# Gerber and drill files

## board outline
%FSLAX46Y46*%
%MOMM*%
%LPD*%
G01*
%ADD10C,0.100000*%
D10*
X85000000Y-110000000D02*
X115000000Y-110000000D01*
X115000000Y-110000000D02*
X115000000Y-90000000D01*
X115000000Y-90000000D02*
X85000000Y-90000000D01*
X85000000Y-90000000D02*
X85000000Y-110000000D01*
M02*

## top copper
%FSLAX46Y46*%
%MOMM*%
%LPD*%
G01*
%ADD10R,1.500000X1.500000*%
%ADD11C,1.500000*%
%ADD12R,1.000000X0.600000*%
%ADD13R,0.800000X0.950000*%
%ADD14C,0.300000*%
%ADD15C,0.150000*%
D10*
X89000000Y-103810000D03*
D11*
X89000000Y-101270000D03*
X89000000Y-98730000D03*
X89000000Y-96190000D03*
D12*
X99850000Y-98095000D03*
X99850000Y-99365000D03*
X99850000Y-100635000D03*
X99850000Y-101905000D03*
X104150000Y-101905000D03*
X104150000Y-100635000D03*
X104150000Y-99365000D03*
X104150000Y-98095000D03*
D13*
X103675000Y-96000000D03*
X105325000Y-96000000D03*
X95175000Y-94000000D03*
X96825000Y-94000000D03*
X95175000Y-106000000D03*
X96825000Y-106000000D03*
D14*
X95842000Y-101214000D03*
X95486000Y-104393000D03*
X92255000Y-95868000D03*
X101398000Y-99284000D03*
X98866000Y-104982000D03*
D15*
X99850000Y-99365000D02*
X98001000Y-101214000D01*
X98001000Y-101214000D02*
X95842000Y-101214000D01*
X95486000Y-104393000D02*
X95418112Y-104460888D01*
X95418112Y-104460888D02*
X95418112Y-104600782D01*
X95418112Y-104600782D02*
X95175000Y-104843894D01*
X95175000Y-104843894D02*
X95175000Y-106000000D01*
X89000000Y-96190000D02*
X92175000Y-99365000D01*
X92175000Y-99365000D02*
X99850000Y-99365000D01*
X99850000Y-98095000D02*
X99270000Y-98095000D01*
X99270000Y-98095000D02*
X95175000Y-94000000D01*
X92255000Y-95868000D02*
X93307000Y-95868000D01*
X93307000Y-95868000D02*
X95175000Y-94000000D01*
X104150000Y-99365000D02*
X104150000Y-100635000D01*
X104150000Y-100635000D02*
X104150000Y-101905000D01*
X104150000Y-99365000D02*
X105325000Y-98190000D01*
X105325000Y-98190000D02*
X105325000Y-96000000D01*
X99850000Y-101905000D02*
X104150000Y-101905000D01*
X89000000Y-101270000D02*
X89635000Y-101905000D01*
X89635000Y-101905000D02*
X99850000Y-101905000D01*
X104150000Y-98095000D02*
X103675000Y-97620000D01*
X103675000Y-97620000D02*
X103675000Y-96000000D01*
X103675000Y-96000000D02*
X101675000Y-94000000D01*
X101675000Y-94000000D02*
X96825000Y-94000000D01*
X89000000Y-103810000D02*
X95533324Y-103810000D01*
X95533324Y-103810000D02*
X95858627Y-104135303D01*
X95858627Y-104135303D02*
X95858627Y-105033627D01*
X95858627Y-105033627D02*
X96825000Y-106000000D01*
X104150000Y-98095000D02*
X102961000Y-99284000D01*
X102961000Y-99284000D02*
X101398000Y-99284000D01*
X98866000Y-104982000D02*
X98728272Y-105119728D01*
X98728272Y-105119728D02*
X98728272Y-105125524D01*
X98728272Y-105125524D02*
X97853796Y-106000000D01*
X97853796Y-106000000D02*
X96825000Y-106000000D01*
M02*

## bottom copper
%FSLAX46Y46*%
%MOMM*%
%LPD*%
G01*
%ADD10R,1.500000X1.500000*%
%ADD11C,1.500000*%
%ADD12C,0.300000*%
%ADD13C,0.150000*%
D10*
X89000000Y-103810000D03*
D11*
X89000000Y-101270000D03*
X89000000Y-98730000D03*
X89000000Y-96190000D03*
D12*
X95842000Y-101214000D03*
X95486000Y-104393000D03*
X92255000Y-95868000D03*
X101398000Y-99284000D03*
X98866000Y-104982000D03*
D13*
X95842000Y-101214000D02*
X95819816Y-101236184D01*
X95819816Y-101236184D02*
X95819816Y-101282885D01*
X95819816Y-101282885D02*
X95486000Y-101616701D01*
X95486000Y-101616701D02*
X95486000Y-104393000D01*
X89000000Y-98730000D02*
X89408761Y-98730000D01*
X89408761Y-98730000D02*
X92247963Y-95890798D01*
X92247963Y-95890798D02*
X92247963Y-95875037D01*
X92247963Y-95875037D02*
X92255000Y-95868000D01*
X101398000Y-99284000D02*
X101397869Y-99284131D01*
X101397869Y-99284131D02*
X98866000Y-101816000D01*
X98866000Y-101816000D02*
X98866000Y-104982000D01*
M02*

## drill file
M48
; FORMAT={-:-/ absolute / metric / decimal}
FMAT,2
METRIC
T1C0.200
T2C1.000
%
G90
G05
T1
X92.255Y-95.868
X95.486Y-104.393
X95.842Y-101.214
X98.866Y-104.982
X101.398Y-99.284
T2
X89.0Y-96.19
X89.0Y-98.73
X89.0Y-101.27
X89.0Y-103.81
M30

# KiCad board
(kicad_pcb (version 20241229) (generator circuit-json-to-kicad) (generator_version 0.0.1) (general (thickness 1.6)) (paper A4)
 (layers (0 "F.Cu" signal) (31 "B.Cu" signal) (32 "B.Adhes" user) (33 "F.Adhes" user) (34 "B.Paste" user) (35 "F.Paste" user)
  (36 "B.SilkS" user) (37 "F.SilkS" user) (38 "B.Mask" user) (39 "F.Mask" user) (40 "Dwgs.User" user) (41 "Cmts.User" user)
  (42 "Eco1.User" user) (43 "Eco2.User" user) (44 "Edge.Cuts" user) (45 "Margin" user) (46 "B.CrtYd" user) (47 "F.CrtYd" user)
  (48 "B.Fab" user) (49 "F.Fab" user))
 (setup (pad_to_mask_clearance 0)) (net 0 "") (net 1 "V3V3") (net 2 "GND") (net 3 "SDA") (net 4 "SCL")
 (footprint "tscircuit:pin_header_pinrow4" (layer F.Cu) (at 89 100 90)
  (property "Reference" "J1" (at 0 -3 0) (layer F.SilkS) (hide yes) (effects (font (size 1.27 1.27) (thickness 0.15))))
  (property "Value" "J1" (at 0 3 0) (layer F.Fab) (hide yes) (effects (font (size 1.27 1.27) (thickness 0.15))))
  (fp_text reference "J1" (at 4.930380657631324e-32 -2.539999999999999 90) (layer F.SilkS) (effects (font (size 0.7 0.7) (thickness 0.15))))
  (pad "1" thru_hole rect (at -3.81 2.3329521523757077e-16 90) (size 1.5 1.5) (drill 1) (layers *.Cu *.Mask) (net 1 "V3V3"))
  (pad "2" thru_hole circle (at -1.27 7.776507174585693e-17 0) (size 1.5 1.5) (drill 1) (layers *.Cu *.Mask) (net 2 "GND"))
  (pad "3" thru_hole circle (at 1.27 -7.776507174585693e-17 0) (size 1.5 1.5) (drill 1) (layers *.Cu *.Mask) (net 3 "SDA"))
  (pad "4" thru_hole circle (at 3.81 -2.3329521523757077e-16 0) (size 1.5 1.5) (drill 1) (layers *.Cu *.Mask) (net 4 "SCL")))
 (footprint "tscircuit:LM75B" (layer F.Cu) (at 102 100 0)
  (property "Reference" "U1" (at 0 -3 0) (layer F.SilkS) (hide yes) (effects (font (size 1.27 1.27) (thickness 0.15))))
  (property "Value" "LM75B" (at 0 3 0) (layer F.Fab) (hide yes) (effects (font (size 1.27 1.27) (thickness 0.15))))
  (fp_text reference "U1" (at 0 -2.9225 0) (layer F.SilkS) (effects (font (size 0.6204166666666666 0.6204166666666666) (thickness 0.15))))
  (pad "1" smd rect (at -2.15 -1.905 0) (size 1 0.6) (layers F.Cu F.Paste F.Mask) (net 3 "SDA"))
  (pad "2" smd rect (at -2.15 -0.635 0) (size 1 0.6) (layers F.Cu F.Paste F.Mask) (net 4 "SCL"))
  (pad "3" smd rect (at -2.15 0.635 0) (size 1 0.6) (layers F.Cu F.Paste F.Mask))
  (pad "4" smd rect (at -2.15 1.905 0) (size 1 0.6) (layers F.Cu F.Paste F.Mask) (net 2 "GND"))
  (pad "5" smd rect (at 2.1500000000000004 1.905 0) (size 1 0.6) (layers F.Cu F.Paste F.Mask) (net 2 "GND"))
  (pad "6" smd rect (at 2.1500000000000004 0.635 0) (size 1 0.6) (layers F.Cu F.Paste F.Mask) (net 2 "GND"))
  (pad "7" smd rect (at 2.1500000000000004 -0.635 0) (size 1 0.6) (layers F.Cu F.Paste F.Mask) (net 2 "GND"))
  (pad "8" smd rect (at 2.1500000000000004 -1.905 0) (size 1 0.6) (layers F.Cu F.Paste F.Mask) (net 1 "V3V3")))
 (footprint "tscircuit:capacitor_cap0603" (layer F.Cu) (at 104.5 96 0)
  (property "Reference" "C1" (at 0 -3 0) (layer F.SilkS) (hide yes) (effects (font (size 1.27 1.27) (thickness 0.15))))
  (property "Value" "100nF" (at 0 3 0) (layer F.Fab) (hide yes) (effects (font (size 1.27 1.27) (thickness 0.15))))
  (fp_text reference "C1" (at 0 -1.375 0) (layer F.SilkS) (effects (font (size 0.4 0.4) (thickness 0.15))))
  (pad "1" smd rect (at -0.8250000000000002 0 0) (size 0.8 0.95) (layers F.Cu F.Paste F.Mask) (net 1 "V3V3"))
  (pad "2" smd rect (at 0.8250000000000002 0 0) (size 0.8 0.95) (layers F.Cu F.Paste F.Mask) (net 2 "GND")))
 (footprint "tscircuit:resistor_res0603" (layer F.Cu) (at 96 94 0)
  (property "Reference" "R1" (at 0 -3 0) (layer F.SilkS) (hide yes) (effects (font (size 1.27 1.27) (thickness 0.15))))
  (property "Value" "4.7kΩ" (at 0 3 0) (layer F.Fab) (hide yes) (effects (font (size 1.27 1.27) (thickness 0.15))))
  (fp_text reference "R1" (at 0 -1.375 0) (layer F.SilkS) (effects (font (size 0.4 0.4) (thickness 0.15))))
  (pad "1" smd rect (at -0.8250000000000002 0 0) (size 0.8 0.95) (layers F.Cu F.Paste F.Mask) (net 3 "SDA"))
  (pad "2" smd rect (at 0.8250000000000002 0 0) (size 0.8 0.95) (layers F.Cu F.Paste F.Mask) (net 1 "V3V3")))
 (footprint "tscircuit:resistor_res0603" (layer F.Cu) (at 96 106 0)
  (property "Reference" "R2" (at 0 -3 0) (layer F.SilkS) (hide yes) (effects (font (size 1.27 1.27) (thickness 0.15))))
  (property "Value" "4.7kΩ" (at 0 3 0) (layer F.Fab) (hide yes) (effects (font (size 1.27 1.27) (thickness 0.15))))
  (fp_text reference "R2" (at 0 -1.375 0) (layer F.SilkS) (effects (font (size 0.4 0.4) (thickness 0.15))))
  (pad "1" smd rect (at -0.8250000000000002 0 0) (size 0.8 0.95) (layers F.Cu F.Paste F.Mask) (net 4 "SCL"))
  (pad "2" smd rect (at 0.8250000000000002 0 0) (size 0.8 0.95) (layers F.Cu F.Paste F.Mask) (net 1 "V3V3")))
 (segment (start 99.85 99.365) (end 98.001 101.214) (width 0.15) (layer F.Cu) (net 4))
 (segment (start 98.001 101.214) (end 95.842 101.214) (width 0.15) (layer F.Cu) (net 4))
 (segment (start 95.842 101.214) (end 95.81981559401727 101.23618440598273) (width 0.15) (layer B.Cu) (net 4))
 (segment (start 95.81981559401727 101.23618440598273) (end 95.81981559401727 101.28288511764556) (width 0.15) (layer B.Cu) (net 4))
 (segment (start 95.81981559401727 101.28288511764556) (end 95.486 101.61670071166283) (width 0.15) (layer B.Cu) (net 4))
 (segment (start 95.486 101.61670071166283) (end 95.486 104.393) (width 0.15) (layer B.Cu) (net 4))
 (segment (start 95.486 104.393) (end 95.41811191088075 104.46088808911925) (width 0.15) (layer F.Cu) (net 4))
 (segment (start 95.41811191088075 104.46088808911925) (end 95.41811191088075 104.60078196186367) (width 0.15) (layer F.Cu) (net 4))
 (segment (start 95.41811191088075 104.60078196186367) (end 95.175 104.84389387274443) (width 0.15) (layer F.Cu) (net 4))
 (segment (start 95.175 104.84389387274443) (end 95.175 106) (width 0.15) (layer F.Cu) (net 4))
 (segment (start 89 96.19) (end 92.175 99.365) (width 0.15) (layer F.Cu) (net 4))
 (segment (start 92.175 99.365) (end 99.85 99.365) (width 0.15) (layer F.Cu) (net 4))
 (segment (start 99.85 98.095) (end 99.27 98.095) (width 0.15) (layer F.Cu) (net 3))
 (segment (start 99.27 98.095) (end 95.175 94) (width 0.15) (layer F.Cu) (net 3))
 (segment (start 89 98.73) (end 89.4087611810871 98.73) (width 0.15) (layer B.Cu) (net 3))
 (segment (start 89.4087611810871 98.73) (end 92.24796273861192 95.89079844247519) (width 0.15) (layer B.Cu) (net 3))
 (segment (start 92.24796273861192 95.89079844247519) (end 92.24796273861192 95.87503726138809) (width 0.15) (layer B.Cu) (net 3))
 (segment (start 92.24796273861192 95.87503726138809) (end 92.255 95.868) (width 0.15) (layer B.Cu) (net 3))
 (segment (start 92.255 95.868) (end 93.307 95.868) (width 0.15) (layer F.Cu) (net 3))
 (segment (start 93.307 95.868) (end 95.175 94) (width 0.15) (layer F.Cu) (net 3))
 (segment (start 104.15 99.365) (end 104.15 100.635) (width 0.15) (layer F.Cu) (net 2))
 (segment (start 104.15 100.635) (end 104.15 101.905) (width 0.15) (layer F.Cu) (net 2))
 (segment (start 104.15 99.365) (end 105.325 98.19) (width 0.15) (layer F.Cu) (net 2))
 (segment (start 105.325 98.19) (end 105.325 96) (width 0.15) (layer F.Cu) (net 2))
 (segment (start 99.85 101.905) (end 104.15 101.905) (width 0.15) (layer F.Cu) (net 2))
 (segment (start 89 101.27) (end 89.635 101.905) (width 0.15) (layer F.Cu) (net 2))
 (segment (start 89.635 101.905) (end 99.85 101.905) (width 0.15) (layer F.Cu) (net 2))
 (segment (start 104.15 98.095) (end 103.675 97.62) (width 0.15) (layer F.Cu) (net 1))
 (segment (start 103.675 97.62) (end 103.675 96) (width 0.15) (layer F.Cu) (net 1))
 (segment (start 103.675 96) (end 101.675 94) (width 0.15) (layer F.Cu) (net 1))
 (segment (start 101.675 94) (end 96.825 94) (width 0.15) (layer F.Cu) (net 1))
 (segment (start 89 103.81) (end 95.5333238737182 103.81) (width 0.15) (layer F.Cu) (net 1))
 (segment (start 95.5333238737182 103.81) (end 95.85862733708665 104.13530346336843) (width 0.15) (layer F.Cu) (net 1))
 (segment (start 95.85862733708665 104.13530346336843) (end 95.85862733708665 105.03362733708664) (width 0.15) (layer F.Cu) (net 1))
 (segment (start 95.85862733708665 105.03362733708664) (end 96.825 106) (width 0.15) (layer F.Cu) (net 1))
 (segment (start 104.15 98.095) (end 102.961 99.284) (width 0.15) (layer F.Cu) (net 1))
 (segment (start 102.961 99.284) (end 101.398 99.284) (width 0.15) (layer F.Cu) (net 1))
 (segment (start 101.398 99.284) (end 101.39786876400757 99.28413123599243) (width 0.15) (layer B.Cu) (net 1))
 (segment (start 101.39786876400757 99.28413123599243) (end 98.866 101.816) (width 0.15) (layer B.Cu) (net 1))
 (segment (start 98.866 101.816) (end 98.866 104.982) (width 0.15) (layer B.Cu) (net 1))
 (segment (start 98.866 104.982) (end 98.72827242804924 105.11972757195076) (width 0.15) (layer F.Cu) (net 1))
 (segment (start 98.72827242804924 105.11972757195076) (end 98.72827242804924 105.12552365933615) (width 0.15) (layer F.Cu) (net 1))
 (segment (start 98.72827242804924 105.12552365933615) (end 97.85379608738539 106) (width 0.15) (layer F.Cu) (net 1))
 (segment (start 97.85379608738539 106) (end 96.825 106) (width 0.15) (layer F.Cu) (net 1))
 (gr_line (start 85 110) (end 115 110) (width 0.1) (layer Edge.Cuts))
 (gr_line (start 115 110) (end 115 90) (width 0.1) (layer Edge.Cuts))
 (gr_line (start 115 90) (end 85 90) (width 0.1) (layer Edge.Cuts))
 (gr_line (start 85 90) (end 85 110) (width 0.1) (layer Edge.Cuts))
 (via (at 95.842 101.214) (size 0.3) (drill 0.2) (layers F.Cu B.Cu) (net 4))
 (via (at 95.486 104.393) (size 0.3) (drill 0.2) (layers F.Cu B.Cu) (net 4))
 (via (at 92.255 95.868) (size 0.3) (drill 0.2) (layers F.Cu B.Cu) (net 3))
 (via (at 101.398 99.284) (size 0.3) (drill 0.2) (layers F.Cu B.Cu) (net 1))
 (via (at 98.866 104.982) (size 0.3) (drill 0.2) (layers F.Cu B.Cu) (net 1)))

